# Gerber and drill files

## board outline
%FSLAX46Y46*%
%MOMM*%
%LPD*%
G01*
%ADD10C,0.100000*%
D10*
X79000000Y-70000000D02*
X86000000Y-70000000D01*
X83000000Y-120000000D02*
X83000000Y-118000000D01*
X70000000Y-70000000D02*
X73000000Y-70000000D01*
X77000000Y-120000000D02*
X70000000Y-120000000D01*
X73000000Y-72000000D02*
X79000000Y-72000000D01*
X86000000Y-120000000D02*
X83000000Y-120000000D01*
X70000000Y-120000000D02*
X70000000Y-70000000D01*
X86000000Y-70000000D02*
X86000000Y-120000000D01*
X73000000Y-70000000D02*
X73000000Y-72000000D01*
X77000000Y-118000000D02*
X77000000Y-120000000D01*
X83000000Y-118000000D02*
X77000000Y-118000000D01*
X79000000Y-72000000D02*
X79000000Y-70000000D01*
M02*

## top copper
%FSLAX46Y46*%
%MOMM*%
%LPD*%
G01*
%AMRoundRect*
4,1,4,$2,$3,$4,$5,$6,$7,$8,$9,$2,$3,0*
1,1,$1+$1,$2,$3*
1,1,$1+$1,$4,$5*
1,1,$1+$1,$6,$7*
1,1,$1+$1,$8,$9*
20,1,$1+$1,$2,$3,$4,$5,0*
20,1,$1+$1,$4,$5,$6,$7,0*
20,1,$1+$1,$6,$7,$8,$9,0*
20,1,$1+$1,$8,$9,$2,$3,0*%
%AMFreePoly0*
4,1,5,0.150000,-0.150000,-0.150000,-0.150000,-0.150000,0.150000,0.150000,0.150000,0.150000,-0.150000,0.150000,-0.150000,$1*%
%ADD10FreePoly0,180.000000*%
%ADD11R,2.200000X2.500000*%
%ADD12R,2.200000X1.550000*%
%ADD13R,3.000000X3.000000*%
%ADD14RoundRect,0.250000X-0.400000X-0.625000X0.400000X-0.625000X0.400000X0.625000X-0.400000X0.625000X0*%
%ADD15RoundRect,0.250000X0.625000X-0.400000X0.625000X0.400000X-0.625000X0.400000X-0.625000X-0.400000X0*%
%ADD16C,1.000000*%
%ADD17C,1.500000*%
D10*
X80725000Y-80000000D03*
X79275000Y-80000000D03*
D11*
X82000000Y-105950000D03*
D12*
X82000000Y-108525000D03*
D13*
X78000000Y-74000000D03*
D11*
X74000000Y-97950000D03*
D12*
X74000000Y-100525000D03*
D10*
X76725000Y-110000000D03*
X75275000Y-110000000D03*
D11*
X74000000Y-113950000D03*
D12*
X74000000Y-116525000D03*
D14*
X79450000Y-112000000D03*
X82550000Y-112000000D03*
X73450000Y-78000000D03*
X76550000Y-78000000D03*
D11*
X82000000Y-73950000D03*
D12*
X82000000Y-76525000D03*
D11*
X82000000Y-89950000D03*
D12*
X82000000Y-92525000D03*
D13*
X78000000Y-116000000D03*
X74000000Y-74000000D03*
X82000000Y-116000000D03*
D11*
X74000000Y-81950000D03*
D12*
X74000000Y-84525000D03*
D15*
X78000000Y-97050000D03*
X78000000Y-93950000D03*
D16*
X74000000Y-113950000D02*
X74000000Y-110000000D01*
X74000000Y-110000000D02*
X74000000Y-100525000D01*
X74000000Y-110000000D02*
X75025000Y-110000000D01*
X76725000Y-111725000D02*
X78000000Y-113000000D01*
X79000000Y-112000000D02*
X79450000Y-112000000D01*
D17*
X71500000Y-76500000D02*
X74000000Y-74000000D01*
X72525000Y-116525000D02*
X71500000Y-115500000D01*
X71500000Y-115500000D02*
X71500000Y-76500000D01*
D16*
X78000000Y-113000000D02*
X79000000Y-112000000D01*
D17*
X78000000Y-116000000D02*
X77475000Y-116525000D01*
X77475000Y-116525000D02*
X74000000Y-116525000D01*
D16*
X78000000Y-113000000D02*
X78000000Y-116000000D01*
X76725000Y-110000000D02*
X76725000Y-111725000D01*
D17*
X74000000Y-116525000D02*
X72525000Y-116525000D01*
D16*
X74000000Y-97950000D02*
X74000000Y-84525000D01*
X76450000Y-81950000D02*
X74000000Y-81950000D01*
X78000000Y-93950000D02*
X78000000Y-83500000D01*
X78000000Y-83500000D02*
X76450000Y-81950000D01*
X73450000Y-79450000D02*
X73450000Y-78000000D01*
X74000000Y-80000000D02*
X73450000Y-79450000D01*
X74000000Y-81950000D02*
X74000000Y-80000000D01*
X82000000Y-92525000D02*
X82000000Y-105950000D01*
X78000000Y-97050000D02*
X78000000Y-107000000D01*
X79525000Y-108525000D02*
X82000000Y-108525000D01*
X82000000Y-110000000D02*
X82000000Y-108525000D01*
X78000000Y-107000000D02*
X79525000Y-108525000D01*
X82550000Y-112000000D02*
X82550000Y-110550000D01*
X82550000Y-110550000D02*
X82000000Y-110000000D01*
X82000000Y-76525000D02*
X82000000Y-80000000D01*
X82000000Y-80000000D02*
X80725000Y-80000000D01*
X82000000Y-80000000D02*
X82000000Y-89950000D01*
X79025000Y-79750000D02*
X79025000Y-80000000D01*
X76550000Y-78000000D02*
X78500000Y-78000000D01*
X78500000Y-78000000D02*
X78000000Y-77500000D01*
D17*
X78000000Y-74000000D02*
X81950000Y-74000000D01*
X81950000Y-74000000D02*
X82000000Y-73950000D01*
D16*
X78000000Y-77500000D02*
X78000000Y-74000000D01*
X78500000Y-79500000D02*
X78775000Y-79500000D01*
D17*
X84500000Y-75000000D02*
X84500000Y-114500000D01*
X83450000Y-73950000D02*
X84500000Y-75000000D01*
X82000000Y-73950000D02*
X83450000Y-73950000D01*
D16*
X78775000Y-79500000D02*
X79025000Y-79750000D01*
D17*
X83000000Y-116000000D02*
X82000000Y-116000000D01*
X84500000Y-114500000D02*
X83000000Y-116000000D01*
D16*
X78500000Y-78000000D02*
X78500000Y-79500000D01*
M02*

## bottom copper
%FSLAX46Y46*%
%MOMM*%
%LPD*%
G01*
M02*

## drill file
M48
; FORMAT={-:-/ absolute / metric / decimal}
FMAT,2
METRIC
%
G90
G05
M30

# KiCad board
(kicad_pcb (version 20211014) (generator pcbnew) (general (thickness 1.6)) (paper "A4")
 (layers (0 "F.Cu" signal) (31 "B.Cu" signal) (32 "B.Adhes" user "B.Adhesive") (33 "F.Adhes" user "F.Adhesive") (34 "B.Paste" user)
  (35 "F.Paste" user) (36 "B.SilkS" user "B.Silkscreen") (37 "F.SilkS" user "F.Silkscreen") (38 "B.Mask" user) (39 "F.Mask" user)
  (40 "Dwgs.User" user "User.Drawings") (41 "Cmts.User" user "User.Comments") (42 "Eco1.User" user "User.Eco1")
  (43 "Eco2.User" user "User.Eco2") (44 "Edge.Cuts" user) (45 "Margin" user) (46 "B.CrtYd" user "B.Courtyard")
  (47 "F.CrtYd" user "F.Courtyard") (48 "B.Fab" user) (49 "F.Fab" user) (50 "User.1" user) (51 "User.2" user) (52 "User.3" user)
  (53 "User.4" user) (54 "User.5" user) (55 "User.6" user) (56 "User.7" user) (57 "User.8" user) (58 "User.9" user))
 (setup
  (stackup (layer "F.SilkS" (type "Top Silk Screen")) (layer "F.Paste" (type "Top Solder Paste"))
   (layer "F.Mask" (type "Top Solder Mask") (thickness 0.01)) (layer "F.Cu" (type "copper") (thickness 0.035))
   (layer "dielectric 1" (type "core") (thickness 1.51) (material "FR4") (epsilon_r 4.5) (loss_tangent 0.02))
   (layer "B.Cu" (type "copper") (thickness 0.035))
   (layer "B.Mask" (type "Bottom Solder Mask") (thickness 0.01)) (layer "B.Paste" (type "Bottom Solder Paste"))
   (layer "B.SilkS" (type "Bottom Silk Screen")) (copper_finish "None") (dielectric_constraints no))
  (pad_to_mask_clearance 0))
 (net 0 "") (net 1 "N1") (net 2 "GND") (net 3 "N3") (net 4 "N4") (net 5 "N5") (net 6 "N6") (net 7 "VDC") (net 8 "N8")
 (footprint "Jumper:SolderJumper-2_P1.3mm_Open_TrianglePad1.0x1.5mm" (layer "F.Cu") (at 80 80 180)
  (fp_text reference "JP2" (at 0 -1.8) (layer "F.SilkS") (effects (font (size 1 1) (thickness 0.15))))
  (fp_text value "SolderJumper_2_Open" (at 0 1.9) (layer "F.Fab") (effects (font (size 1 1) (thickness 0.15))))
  (pad "1" smd custom (at -0.725 0 180) (size 0.3 0.3) (layers "F.Cu" "F.Mask") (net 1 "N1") (zone_connect 2)
   (options (clearance outline) (anchor rect)) (primitives))
  (pad "2" smd custom (at 0.725 0 180) (size 0.3 0.3) (layers "F.Cu" "F.Mask") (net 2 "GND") (zone_connect 2)
   (options (clearance outline) (anchor rect)) (primitives)))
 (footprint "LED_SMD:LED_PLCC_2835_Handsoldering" (layer "F.Cu") (at 82 107 -90)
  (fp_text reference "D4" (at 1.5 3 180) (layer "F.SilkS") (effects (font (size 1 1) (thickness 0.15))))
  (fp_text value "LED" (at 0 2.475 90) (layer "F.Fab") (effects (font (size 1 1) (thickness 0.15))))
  (pad "1" smd rect (at -1.05 0 270) (size 2.5 2.2) (layers "F.Cu" "F.Paste" "F.Mask") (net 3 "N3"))
  (pad "2" smd rect (at 1.525 0 270) (size 1.55 2.2) (layers "F.Cu" "F.Paste" "F.Mask") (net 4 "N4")))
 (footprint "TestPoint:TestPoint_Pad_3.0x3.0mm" (layer "F.Cu") (at 78 74)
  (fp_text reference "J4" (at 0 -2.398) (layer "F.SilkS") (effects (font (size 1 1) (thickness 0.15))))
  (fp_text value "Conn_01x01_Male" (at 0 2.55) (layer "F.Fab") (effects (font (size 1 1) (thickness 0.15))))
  (pad "1" smd rect (at 0 0) (size 3 3) (layers "F.Cu" "F.Mask") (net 2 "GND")))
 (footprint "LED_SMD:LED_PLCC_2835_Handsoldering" (layer "F.Cu") (at 74 99 -90)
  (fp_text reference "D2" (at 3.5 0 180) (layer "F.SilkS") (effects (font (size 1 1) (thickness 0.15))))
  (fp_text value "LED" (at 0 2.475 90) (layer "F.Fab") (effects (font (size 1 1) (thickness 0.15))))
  (pad "1" smd rect (at -1.05 0 270) (size 2.5 2.2) (layers "F.Cu" "F.Paste" "F.Mask") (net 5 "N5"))
  (pad "2" smd rect (at 1.525 0 270) (size 1.55 2.2) (layers "F.Cu" "F.Paste" "F.Mask") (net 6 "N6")))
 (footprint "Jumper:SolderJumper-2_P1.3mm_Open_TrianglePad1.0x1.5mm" (layer "F.Cu") (at 76 110 180)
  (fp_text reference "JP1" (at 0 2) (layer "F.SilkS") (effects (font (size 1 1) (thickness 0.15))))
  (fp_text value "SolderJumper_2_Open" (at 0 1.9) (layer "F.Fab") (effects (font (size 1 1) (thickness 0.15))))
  (pad "1" smd custom (at -0.725 0 180) (size 0.3 0.3) (layers "F.Cu" "F.Mask") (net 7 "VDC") (zone_connect 2)
   (options (clearance outline) (anchor rect)) (primitives))
  (pad "2" smd custom (at 0.725 0 180) (size 0.3 0.3) (layers "F.Cu" "F.Mask") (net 6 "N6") (zone_connect 2)
   (options (clearance outline) (anchor rect)) (primitives)))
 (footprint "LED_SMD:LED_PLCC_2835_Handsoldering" (layer "F.Cu") (at 74 115 -90)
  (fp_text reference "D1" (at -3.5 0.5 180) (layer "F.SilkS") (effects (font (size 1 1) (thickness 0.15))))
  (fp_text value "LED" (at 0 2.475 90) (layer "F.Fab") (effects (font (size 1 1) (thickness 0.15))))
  (pad "1" smd rect (at -1.05 0 270) (size 2.5 2.2) (layers "F.Cu" "F.Paste" "F.Mask") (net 6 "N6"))
  (pad "2" smd rect (at 1.525 0 270) (size 1.55 2.2) (layers "F.Cu" "F.Paste" "F.Mask") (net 7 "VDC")))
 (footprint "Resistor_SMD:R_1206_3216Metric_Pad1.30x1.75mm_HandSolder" (layer "F.Cu") (at 81 112)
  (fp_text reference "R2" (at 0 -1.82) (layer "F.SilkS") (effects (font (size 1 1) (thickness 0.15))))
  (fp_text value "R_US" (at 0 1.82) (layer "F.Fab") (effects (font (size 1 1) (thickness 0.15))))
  (pad "1" smd roundrect (at -1.55 0) (size 1.3 1.75) (layers "F.Cu" "F.Paste" "F.Mask") (roundrect_rratio 0.192308) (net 7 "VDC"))
  (pad "2" smd roundrect (at 1.55 0) (size 1.3 1.75) (layers "F.Cu" "F.Paste" "F.Mask") (roundrect_rratio 0.192308) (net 4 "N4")))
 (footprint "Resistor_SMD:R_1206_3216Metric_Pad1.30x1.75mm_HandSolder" (layer "F.Cu") (at 75 78)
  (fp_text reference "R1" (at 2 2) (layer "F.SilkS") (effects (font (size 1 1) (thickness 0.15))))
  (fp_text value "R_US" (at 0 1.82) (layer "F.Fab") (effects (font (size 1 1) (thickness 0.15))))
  (pad "1" smd roundrect (at -1.55 0) (size 1.3 1.75) (layers "F.Cu" "F.Paste" "F.Mask") (roundrect_rratio 0.192308) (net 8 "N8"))
  (pad "2" smd roundrect (at 1.55 0) (size 1.3 1.75) (layers "F.Cu" "F.Paste" "F.Mask") (roundrect_rratio 0.192308) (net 2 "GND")))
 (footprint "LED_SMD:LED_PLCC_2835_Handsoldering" (layer "F.Cu") (at 82 75 -90)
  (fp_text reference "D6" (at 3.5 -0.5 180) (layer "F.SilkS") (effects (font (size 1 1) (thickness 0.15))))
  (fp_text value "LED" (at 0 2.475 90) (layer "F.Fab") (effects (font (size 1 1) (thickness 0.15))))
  (pad "1" smd rect (at -1.05 0 270) (size 2.5 2.2) (layers "F.Cu" "F.Paste" "F.Mask") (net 2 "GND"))
  (pad "2" smd rect (at 1.525 0 270) (size 1.55 2.2) (layers "F.Cu" "F.Paste" "F.Mask") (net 1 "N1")))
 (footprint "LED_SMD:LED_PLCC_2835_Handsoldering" (layer "F.Cu") (at 82 91 -90)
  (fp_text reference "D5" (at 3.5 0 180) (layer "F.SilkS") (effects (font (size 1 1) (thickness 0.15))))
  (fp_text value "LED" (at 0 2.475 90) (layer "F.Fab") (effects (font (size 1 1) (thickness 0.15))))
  (pad "1" smd rect (at -1.05 0 270) (size 2.5 2.2) (layers "F.Cu" "F.Paste" "F.Mask") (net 1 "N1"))
  (pad "2" smd rect (at 1.525 0 270) (size 1.55 2.2) (layers "F.Cu" "F.Paste" "F.Mask") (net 3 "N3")))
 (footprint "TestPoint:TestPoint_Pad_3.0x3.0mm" (layer "F.Cu") (at 78 116)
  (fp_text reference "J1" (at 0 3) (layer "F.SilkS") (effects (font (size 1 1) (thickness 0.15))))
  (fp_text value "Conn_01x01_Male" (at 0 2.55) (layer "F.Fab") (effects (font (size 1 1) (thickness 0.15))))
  (pad "1" smd rect (at 0 0) (size 3 3) (layers "F.Cu" "F.Mask") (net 7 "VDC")))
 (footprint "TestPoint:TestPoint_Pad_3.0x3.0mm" (layer "F.Cu") (at 74 74)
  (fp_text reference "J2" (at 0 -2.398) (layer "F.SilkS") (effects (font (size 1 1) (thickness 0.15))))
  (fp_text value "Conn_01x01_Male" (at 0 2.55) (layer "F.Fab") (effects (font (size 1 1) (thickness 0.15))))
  (pad "1" smd rect (at 0 0) (size 3 3) (layers "F.Cu" "F.Mask") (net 7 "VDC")))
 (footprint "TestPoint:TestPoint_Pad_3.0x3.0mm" (layer "F.Cu") (at 82 116)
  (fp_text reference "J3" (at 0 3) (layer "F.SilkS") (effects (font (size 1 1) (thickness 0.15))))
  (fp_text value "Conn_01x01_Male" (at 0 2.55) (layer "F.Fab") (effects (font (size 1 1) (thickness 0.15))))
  (pad "1" smd rect (at 0 0) (size 3 3) (layers "F.Cu" "F.Mask") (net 2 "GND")))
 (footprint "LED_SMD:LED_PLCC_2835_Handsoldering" (layer "F.Cu") (at 74 83 -90)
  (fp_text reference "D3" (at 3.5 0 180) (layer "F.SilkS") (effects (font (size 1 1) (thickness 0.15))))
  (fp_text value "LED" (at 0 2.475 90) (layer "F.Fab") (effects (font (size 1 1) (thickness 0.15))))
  (pad "1" smd rect (at -1.05 0 270) (size 2.5 2.2) (layers "F.Cu" "F.Paste" "F.Mask") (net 8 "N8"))
  (pad "2" smd rect (at 1.525 0 270) (size 1.55 2.2) (layers "F.Cu" "F.Paste" "F.Mask") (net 5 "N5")))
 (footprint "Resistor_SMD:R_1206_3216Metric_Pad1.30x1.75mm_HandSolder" (layer "F.Cu") (at 78 95.5 90)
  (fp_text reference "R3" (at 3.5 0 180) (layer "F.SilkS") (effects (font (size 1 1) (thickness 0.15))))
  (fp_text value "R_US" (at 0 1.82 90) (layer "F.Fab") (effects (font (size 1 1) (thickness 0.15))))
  (pad "1" smd roundrect (at -1.55 0 90) (size 1.3 1.75) (layers "F.Cu" "F.Paste" "F.Mask") (roundrect_rratio 0.192308) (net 4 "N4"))
  (pad "2" smd roundrect (at 1.55 0 90) (size 1.3 1.75) (layers "F.Cu" "F.Paste" "F.Mask") (roundrect_rratio 0.192308) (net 8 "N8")))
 (gr_line (start 79 70) (end 86 70) (layer "Edge.Cuts") (width 0.1))
 (gr_line (start 83 120) (end 83 118) (layer "Edge.Cuts") (width 0.1))
 (gr_line (start 70 70) (end 73 70) (layer "Edge.Cuts") (width 0.1))
 (gr_line (start 77 120) (end 70 120) (layer "Edge.Cuts") (width 0.1))
 (gr_line (start 73 72) (end 79 72) (layer "Edge.Cuts") (width 0.1))
 (gr_line (start 86 120) (end 83 120) (layer "Edge.Cuts") (width 0.1))
 (gr_line (start 70 120) (end 70 70) (layer "Edge.Cuts") (width 0.1))
 (gr_line (start 86 70) (end 86 120) (layer "Edge.Cuts") (width 0.1))
 (gr_line (start 73 70) (end 73 72) (layer "Edge.Cuts") (width 0.1))
 (gr_line (start 77 118) (end 77 120) (layer "Edge.Cuts") (width 0.1))
 (gr_line (start 83 118) (end 77 118) (layer "Edge.Cuts") (width 0.1))
 (gr_line (start 79 72) (end 79 70) (layer "Edge.Cuts") (width 0.1))
 (segment (start 74 113.95) (end 74 110) (width 1) (layer "F.Cu") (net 6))
 (segment (start 74 110) (end 74 100.525) (width 1) (layer "F.Cu") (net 6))
 (segment (start 74 110) (end 75.025 110) (width 1) (layer "F.Cu") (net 6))
 (segment (start 76.725 111.725) (end 78 113) (width 1) (layer "F.Cu") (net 7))
 (segment (start 79 112) (end 79.45 112) (width 1) (layer "F.Cu") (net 7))
 (segment (start 71.5 76.5) (end 74 74) (width 1.5) (layer "F.Cu") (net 7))
 (segment (start 72.525 116.525) (end 71.5 115.5) (width 1.5) (layer "F.Cu") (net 7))
 (segment (start 71.5 115.5) (end 71.5 76.5) (width 1.5) (layer "F.Cu") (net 7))
 (segment (start 78 113) (end 79 112) (width 1) (layer "F.Cu") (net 7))
 (segment (start 78 116) (end 77.475 116.525) (width 1.5) (layer "F.Cu") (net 7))
 (segment (start 77.475 116.525) (end 74 116.525) (width 1.5) (layer "F.Cu") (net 7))
 (segment (start 78 113) (end 78 116) (width 1) (layer "F.Cu") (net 7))
 (segment (start 76.725 110) (end 76.725 111.725) (width 1) (layer "F.Cu") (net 7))
 (segment (start 74 116.525) (end 72.525 116.525) (width 1.5) (layer "F.Cu") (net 7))
 (segment (start 74 97.95) (end 74 84.525) (width 1) (layer "F.Cu") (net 5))
 (segment (start 76.45 81.95) (end 74 81.95) (width 1) (layer "F.Cu") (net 8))
 (segment (start 78 93.95) (end 78 83.5) (width 1) (layer "F.Cu") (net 8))
 (segment (start 78 83.5) (end 76.45 81.95) (width 1) (layer "F.Cu") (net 8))
 (segment (start 73.45 79.45) (end 73.45 78) (width 1) (layer "F.Cu") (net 8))
 (segment (start 74 80) (end 73.45 79.45) (width 1) (layer "F.Cu") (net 8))
 (segment (start 74 81.95) (end 74 80) (width 1) (layer "F.Cu") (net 8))
 (segment (start 82 92.525) (end 82 105.95) (width 1) (layer "F.Cu") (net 3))
 (segment (start 78 97.05) (end 78 107) (width 1) (layer "F.Cu") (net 4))
 (segment (start 79.525 108.525) (end 82 108.525) (width 1) (layer "F.Cu") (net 4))
 (segment (start 82 110) (end 82 108.525) (width 1) (layer "F.Cu") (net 4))
 (segment (start 78 107) (end 79.525 108.525) (width 1) (layer "F.Cu") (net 4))
 (segment (start 82.55 112) (end 82.55 110.55) (width 1) (layer "F.Cu") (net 4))
 (segment (start 82.55 110.55) (end 82 110) (width 1) (layer "F.Cu") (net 4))
 (segment (start 82 76.525) (end 82 80) (width 1) (layer "F.Cu") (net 1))
 (segment (start 82 80) (end 80.725 80) (width 1) (layer "F.Cu") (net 1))
 (segment (start 82 80) (end 82 89.95) (width 1) (layer "F.Cu") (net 1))
 (segment (start 79.025 79.75) (end 79.025 80) (width 1) (layer "F.Cu") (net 2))
 (segment (start 76.55 78) (end 78.5 78) (width 1) (layer "F.Cu") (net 2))
 (segment (start 78.5 78) (end 78 77.5) (width 1) (layer "F.Cu") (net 2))
 (segment (start 78 74) (end 81.95 74) (width 1.5) (layer "F.Cu") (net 2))
 (segment (start 81.95 74) (end 82 73.95) (width 1.5) (layer "F.Cu") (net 2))
 (segment (start 78 77.5) (end 78 74) (width 1) (layer "F.Cu") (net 2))
 (segment (start 78.5 79.5) (end 78.775 79.5) (width 1) (layer "F.Cu") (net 2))
 (segment (start 84.5 75) (end 84.5 114.5) (width 1.5) (layer "F.Cu") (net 2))
 (segment (start 83.45 73.95) (end 84.5 75) (width 1.5) (layer "F.Cu") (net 2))
 (segment (start 82 73.95) (end 83.45 73.95) (width 1.5) (layer "F.Cu") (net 2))
 (segment (start 78.775 79.5) (end 79.025 79.75) (width 1) (layer "F.Cu") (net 2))
 (segment (start 83 116) (end 82 116) (width 1.5) (layer "F.Cu") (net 2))
 (segment (start 84.5 114.5) (end 83 116) (width 1.5) (layer "F.Cu") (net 2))
 (segment (start 78.5 78) (end 78.5 79.5) (width 1) (layer "F.Cu") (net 2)))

